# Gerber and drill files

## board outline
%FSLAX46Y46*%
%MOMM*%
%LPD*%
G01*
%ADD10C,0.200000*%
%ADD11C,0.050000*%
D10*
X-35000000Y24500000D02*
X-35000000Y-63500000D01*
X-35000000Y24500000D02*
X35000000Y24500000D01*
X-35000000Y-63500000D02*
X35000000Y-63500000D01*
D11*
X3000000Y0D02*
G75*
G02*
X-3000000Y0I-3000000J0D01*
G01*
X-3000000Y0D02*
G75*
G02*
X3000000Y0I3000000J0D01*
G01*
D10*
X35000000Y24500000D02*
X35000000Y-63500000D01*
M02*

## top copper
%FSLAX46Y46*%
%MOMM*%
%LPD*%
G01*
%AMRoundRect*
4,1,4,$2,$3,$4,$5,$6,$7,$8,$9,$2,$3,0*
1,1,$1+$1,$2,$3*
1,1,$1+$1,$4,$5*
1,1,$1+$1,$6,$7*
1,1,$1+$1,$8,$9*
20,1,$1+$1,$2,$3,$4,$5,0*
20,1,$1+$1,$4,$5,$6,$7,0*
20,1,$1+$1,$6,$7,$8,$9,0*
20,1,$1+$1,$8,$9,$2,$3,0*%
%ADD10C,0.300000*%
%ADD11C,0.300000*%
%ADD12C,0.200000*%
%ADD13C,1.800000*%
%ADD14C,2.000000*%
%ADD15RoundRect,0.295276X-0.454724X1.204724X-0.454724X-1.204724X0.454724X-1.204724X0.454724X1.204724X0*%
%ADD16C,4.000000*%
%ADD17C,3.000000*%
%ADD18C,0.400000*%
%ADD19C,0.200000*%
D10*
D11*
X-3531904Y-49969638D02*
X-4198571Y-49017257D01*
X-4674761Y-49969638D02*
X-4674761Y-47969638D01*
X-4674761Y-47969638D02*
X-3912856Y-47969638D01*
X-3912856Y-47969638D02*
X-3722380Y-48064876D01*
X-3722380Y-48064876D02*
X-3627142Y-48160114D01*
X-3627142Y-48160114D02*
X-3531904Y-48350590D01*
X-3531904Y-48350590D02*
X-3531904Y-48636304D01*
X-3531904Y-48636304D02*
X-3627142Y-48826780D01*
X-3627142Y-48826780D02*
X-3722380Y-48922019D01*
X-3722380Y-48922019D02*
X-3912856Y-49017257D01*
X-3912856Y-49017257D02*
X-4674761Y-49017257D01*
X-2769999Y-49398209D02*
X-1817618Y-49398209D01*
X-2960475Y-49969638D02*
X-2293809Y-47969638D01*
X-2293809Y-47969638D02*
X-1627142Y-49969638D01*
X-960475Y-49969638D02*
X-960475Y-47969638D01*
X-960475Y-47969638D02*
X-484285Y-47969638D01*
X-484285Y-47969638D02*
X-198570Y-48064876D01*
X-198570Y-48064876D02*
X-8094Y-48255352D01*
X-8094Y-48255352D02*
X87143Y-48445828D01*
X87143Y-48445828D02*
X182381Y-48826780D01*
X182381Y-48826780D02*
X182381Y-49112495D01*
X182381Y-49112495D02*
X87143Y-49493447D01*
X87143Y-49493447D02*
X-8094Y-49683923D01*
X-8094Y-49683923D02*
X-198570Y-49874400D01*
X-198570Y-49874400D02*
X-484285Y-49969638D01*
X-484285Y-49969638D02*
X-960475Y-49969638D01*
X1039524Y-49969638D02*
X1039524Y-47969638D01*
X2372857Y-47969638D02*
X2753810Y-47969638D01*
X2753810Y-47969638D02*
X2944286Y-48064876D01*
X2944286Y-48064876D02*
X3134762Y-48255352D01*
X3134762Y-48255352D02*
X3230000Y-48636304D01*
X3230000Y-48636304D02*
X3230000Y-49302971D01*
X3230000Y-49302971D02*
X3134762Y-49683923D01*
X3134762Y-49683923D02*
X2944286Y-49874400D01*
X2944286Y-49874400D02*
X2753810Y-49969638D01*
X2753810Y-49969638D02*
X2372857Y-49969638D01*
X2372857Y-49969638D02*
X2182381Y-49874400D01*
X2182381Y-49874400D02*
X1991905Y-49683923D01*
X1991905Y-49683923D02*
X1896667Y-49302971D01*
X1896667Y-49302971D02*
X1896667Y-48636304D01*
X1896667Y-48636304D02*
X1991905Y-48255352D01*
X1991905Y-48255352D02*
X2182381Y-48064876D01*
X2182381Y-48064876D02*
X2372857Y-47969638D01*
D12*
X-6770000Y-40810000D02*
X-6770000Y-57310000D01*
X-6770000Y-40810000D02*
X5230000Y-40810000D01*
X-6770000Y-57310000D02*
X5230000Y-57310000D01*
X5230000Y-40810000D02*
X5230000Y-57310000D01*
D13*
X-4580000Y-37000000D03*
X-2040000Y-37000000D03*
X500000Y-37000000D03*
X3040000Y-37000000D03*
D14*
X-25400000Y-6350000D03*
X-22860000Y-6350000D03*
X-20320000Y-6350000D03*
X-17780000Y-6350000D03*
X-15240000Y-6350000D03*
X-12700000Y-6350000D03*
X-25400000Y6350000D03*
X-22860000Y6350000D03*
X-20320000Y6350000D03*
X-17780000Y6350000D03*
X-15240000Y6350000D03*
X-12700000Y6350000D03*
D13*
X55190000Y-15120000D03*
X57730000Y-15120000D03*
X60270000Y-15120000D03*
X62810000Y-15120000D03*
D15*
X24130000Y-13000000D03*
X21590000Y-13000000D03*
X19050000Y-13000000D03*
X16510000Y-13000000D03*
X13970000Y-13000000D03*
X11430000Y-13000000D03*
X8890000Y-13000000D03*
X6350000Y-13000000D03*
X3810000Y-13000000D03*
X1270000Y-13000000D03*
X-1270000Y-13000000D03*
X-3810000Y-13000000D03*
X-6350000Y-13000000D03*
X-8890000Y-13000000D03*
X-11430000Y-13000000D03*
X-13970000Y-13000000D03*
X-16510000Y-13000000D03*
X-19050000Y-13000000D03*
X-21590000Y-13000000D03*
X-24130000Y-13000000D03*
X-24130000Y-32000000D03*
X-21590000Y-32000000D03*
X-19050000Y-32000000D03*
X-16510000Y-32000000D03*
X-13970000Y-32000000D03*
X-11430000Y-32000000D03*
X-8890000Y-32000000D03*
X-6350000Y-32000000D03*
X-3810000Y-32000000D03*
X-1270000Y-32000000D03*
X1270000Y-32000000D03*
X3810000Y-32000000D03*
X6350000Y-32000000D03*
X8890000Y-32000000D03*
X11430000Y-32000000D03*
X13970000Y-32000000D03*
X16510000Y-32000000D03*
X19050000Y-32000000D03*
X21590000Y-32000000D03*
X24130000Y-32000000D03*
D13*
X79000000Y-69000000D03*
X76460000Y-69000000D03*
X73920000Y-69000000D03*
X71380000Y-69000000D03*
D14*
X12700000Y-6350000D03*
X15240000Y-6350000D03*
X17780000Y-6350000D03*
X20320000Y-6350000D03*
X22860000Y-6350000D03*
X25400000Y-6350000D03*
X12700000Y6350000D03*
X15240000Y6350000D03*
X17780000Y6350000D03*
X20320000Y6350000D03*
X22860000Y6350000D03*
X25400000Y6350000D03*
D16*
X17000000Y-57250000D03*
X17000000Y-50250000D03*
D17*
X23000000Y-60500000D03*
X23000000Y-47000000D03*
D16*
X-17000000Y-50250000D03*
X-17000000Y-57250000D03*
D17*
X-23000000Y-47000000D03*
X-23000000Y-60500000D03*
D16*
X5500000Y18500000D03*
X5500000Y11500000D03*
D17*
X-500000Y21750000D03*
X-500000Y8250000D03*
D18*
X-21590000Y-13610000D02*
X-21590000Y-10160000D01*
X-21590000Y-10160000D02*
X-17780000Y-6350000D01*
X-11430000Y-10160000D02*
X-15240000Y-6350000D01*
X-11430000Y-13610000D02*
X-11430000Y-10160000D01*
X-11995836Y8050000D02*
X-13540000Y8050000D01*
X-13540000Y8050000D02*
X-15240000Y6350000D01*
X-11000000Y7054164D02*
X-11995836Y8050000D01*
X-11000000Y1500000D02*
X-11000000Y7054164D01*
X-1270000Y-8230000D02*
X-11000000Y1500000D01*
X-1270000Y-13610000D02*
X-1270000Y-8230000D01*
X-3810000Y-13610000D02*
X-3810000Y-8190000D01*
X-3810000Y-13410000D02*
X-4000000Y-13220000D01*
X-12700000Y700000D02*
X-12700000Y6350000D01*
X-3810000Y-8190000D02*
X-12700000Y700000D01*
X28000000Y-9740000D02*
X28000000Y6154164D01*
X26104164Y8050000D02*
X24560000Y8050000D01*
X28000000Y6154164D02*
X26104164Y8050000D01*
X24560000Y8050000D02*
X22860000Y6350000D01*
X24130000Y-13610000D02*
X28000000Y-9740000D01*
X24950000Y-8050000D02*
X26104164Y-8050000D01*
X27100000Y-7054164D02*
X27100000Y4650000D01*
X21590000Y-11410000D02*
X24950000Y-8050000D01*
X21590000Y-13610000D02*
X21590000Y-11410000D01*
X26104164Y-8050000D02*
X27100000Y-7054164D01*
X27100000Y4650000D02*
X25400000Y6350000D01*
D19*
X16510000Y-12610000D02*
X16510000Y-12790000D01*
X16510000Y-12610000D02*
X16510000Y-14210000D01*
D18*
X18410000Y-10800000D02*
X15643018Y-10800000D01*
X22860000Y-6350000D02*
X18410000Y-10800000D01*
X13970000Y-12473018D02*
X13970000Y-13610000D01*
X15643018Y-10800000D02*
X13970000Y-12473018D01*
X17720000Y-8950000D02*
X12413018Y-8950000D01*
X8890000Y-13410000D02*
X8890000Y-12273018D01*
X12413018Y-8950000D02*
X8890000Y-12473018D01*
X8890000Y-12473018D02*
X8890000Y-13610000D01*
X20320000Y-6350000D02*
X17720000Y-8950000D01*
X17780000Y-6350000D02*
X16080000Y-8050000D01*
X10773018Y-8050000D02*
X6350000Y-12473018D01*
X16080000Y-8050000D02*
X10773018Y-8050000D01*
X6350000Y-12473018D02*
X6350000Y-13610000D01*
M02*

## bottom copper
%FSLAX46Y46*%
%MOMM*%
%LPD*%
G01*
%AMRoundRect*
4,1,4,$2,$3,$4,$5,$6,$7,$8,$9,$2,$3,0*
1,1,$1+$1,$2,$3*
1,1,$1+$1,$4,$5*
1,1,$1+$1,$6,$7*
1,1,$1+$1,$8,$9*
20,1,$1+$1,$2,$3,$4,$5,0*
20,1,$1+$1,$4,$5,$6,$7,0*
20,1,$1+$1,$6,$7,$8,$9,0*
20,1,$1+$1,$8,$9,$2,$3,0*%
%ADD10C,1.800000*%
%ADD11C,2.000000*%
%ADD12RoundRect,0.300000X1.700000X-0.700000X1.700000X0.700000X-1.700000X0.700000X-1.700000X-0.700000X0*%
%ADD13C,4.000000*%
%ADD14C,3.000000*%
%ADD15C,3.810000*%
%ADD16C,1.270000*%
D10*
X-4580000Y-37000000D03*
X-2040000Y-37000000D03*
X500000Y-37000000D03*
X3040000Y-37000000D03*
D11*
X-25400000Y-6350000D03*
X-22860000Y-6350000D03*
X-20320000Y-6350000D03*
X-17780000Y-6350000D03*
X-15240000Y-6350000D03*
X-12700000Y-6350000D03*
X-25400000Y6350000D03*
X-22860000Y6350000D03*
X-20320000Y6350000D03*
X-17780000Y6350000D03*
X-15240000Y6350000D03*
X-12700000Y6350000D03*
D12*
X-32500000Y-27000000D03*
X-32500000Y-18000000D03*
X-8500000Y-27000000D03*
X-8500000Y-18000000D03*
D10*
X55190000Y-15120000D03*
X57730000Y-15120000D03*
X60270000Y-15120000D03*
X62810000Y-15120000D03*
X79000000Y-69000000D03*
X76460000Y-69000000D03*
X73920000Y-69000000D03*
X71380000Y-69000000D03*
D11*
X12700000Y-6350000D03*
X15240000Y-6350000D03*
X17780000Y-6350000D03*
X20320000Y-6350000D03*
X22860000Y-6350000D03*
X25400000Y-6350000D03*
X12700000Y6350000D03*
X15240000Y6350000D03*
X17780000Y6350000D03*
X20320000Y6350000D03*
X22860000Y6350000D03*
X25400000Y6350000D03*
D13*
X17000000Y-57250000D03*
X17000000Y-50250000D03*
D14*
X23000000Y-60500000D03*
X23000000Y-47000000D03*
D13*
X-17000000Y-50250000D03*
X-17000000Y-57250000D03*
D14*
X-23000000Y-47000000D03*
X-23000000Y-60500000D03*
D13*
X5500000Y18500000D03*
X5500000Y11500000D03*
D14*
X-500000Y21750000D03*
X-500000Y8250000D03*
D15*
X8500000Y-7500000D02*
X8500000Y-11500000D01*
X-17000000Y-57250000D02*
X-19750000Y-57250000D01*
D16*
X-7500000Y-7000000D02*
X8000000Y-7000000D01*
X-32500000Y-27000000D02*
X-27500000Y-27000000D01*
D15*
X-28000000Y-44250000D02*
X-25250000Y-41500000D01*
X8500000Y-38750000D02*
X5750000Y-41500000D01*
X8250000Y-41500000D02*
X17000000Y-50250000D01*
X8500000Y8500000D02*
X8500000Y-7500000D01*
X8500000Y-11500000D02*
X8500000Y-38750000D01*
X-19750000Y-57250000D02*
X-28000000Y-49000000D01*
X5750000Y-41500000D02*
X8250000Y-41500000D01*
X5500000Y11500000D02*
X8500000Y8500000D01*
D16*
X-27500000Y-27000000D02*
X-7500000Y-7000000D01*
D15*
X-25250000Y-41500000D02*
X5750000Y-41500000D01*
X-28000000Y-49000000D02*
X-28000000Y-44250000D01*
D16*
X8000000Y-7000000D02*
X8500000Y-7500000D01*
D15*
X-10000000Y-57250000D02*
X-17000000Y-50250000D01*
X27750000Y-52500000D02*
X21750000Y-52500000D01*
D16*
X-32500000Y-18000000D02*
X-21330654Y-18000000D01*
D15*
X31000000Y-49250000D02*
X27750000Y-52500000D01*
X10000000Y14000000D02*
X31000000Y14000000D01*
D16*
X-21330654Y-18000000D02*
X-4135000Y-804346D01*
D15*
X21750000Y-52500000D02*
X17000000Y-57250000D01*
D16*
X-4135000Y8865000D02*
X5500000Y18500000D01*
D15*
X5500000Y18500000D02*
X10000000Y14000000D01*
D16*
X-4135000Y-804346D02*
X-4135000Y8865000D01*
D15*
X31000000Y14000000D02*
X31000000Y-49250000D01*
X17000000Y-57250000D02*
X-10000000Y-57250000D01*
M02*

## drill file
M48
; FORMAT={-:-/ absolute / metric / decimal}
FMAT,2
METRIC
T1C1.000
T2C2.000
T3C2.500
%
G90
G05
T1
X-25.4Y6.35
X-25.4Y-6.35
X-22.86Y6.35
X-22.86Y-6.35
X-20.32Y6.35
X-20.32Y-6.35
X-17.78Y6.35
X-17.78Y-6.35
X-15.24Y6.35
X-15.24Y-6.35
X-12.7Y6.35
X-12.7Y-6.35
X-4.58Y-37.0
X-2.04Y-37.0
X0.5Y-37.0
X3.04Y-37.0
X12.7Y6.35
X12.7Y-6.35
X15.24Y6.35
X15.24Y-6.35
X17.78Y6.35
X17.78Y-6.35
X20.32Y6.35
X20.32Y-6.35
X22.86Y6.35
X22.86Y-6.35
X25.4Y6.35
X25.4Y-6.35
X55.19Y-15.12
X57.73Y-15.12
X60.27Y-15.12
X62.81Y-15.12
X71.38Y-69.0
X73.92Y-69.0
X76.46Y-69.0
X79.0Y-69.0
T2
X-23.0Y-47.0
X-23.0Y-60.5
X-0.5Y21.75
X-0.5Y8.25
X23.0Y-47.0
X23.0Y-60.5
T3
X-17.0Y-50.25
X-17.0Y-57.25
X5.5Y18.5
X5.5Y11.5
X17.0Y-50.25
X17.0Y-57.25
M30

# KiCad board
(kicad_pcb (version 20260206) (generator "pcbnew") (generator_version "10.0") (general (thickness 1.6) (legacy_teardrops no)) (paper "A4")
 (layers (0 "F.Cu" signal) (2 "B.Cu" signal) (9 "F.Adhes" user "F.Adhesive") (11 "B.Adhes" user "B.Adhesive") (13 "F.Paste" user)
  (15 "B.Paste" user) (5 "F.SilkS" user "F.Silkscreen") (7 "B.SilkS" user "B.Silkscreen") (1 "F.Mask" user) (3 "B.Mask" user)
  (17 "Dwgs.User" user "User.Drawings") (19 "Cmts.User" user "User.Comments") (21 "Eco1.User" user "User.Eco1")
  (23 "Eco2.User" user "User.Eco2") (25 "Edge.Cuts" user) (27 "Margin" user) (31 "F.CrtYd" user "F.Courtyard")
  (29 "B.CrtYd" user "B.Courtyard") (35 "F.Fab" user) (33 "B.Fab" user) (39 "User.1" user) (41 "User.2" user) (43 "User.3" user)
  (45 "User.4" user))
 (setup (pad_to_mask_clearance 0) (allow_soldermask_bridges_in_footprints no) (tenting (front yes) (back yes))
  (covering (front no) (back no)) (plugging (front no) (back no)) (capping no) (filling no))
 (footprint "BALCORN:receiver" (layer "F.Cu") (at -0.77 49.06)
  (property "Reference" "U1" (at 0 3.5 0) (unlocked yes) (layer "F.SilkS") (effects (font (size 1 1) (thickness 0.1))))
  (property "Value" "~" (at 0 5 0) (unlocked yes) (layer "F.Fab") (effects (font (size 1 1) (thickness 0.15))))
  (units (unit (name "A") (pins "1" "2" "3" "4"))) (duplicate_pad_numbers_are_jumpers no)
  (fp_line (start -6 -8.25) (end -6 8.25) (stroke (width 0.2) (type default)) (layer "F.Cu"))
  (fp_line (start -6 -8.25) (end 6 -8.25) (stroke (width 0.2) (type default)) (layer "F.Cu"))
  (fp_line (start -6 8.25) (end 6 8.25) (stroke (width 0.2) (type default)) (layer "F.Cu"))
  (fp_line (start 6 -8.25) (end 6 8.25) (stroke (width 0.2) (type default)) (layer "F.Cu"))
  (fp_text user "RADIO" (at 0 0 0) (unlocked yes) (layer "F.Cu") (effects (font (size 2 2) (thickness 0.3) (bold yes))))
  (pad "1" thru_hole circle (at -3.81 -12.06) (size 1.8 1.8) (drill 1) (layers "*.Cu" "*.Mask") (remove_unused_layers no)
   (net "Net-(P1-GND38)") (thermal_bridge_angle 90))
  (pad "2" thru_hole circle (at -1.27 -12.06) (size 1.8 1.8) (drill 1) (layers "*.Cu" "*.Mask") (remove_unused_layers no)
   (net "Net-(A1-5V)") (thermal_bridge_angle 90))
  (pad "3" thru_hole circle (at 1.27 -12.06) (size 1.8 1.8) (drill 1) (layers "*.Cu" "*.Mask") (remove_unused_layers no)
   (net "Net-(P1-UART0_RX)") (thermal_bridge_angle 90))
  (pad "4" thru_hole circle (at 3.81 -12.06) (size 1.8 1.8) (drill 1) (layers "*.Cu" "*.Mask") (remove_unused_layers no)
   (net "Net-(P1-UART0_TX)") (thermal_bridge_angle 90)))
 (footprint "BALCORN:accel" (layer "F.Cu") (at -19.05 0 90)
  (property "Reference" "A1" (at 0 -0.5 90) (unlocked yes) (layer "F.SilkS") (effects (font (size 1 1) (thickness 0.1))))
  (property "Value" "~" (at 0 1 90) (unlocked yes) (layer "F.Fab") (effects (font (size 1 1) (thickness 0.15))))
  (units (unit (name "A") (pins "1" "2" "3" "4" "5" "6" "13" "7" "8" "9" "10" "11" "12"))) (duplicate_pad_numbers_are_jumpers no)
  (pad "1" thru_hole circle (at -6.35 -6.35 90) (size 2 2) (drill 1) (layers "*.Cu" "*.Mask") (remove_unused_layers no) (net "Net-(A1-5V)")
   (thermal_bridge_angle 90))
  (pad "2" thru_hole circle (at -6.35 -3.81 90) (size 2 2) (drill 1) (layers "*.Cu" "*.Mask") (remove_unused_layers no)
   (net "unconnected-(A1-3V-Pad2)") (thermal_bridge_angle 90))
  (pad "3" thru_hole circle (at -6.35 -1.27 90) (size 2 2) (drill 1) (layers "*.Cu" "*.Mask") (remove_unused_layers no)
   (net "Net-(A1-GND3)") (thermal_bridge_angle 90))
  (pad "4" thru_hole circle (at -6.35 1.27 90) (size 2 2) (drill 1) (layers "*.Cu" "*.Mask") (remove_unused_layers no) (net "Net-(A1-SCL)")
   (thermal_bridge_angle 90))
  (pad "5" thru_hole circle (at -6.35 3.81 90) (size 2 2) (drill 1) (layers "*.Cu" "*.Mask") (remove_unused_layers no) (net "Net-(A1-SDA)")
   (thermal_bridge_angle 90))
  (pad "6" thru_hole circle (at -6.35 6.35 90) (size 2 2) (drill 1) (layers "*.Cu" "*.Mask") (remove_unused_layers no)
   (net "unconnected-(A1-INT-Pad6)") (thermal_bridge_angle 90))
  (pad "7" thru_hole circle (at 6.35 -6.35 90) (size 2 2) (drill 1) (layers "*.Cu" "*.Mask") (remove_unused_layers no)
   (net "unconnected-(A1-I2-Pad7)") (thermal_bridge_angle 90))
  (pad "8" thru_hole circle (at 6.35 -3.81 90) (size 2 2) (drill 1) (layers "*.Cu" "*.Mask") (remove_unused_layers no)
   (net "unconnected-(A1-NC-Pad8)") (thermal_bridge_angle 90))
  (pad "9" thru_hole circle (at 6.35 -1.27 90) (size 2 2) (drill 1) (layers "*.Cu" "*.Mask") (remove_unused_layers no)
   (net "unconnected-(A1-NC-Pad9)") (thermal_bridge_angle 90))
  (pad "10" thru_hole circle (at 6.35 1.27 90) (size 2 2) (drill 1) (layers "*.Cu" "*.Mask") (remove_unused_layers no)
   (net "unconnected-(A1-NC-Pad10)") (thermal_bridge_angle 90))
  (pad "11" thru_hole circle (at 6.35 3.81 90) (size 2 2) (drill 1) (layers "*.Cu" "*.Mask") (remove_unused_layers no) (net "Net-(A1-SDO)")
   (thermal_bridge_angle 90))
  (pad "12" thru_hole circle (at 6.35 6.35 90) (size 2 2) (drill 1) (layers "*.Cu" "*.Mask") (remove_unused_layers no) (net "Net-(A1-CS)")
   (thermal_bridge_angle 90)))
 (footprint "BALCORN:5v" (layer "F.Cu") (at -20.5 22.5 90)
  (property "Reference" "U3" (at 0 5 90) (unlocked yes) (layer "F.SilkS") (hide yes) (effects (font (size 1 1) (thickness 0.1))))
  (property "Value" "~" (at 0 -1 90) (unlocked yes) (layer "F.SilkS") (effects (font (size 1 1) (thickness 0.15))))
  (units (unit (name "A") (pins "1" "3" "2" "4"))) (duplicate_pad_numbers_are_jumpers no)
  (pad "1" smd roundrect (at -4.5 -12 90) (size 2 4) (layers "B.Cu" "B.Mask") (roundrect_rratio 0.15) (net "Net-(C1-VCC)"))
  (pad "2" smd roundrect (at 4.5 -12 90) (size 2 4) (layers "B.Cu" "B.Mask") (roundrect_rratio 0.15) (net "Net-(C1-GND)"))
  (pad "3" smd roundrect (at -4.5 12 90) (size 2 4) (layers "B.Cu" "B.Mask") (roundrect_rratio 0.15) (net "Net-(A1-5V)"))
  (pad "4" smd roundrect (at 4.5 12 90) (size 2 4) (layers "B.Cu" "B.Mask") (roundrect_rratio 0.15) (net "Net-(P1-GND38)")))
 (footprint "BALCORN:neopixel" (layer "F.Cu") (at 59 15.12)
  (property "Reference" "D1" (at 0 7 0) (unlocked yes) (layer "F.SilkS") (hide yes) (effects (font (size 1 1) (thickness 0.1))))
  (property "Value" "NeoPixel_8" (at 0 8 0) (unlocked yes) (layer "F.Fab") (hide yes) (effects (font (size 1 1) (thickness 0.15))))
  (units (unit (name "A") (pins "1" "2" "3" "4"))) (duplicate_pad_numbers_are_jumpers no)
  (pad "1" thru_hole circle (at -3.81 0) (size 1.8 1.8) (drill 1) (layers "*.Cu" "*.Mask") (remove_unused_layers no)
   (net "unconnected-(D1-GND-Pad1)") (thermal_bridge_angle 90))
  (pad "2" thru_hole circle (at -1.27 0) (size 1.8 1.8) (drill 1) (layers "*.Cu" "*.Mask") (remove_unused_layers no)
   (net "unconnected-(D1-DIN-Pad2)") (thermal_bridge_angle 90))
  (pad "3" thru_hole circle (at 1.27 0) (size 1.8 1.8) (drill 1) (layers "*.Cu" "*.Mask") (remove_unused_layers no) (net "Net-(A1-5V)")
   (thermal_bridge_angle 90))
  (pad "4" thru_hole circle (at 3.81 0) (size 1.8 1.8) (drill 1) (layers "*.Cu" "*.Mask") (remove_unused_layers no) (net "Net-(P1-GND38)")
   (thermal_bridge_angle 90)))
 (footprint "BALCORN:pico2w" (layer "F.Cu") (at 0 22.5 -90)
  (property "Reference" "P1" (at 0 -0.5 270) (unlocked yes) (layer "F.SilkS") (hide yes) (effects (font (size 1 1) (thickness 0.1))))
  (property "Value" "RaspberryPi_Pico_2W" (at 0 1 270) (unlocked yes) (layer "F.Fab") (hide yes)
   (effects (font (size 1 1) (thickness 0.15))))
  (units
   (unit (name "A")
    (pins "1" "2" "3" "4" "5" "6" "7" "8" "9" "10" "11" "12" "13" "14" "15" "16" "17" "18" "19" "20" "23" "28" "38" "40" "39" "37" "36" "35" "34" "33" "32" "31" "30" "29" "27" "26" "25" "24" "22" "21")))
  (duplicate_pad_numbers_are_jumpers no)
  (pad "1" smd roundrect (at -8.89 -24.13 270) (size 3 1.5) (drill (offset -0.61 0)) (layers "F.Cu" "F.Mask")
   (roundrect_rratio 0.1968503937) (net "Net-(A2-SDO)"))
  (pad "2" smd roundrect (at -8.89 -21.59 270) (size 3 1.5) (drill (offset -0.61 0)) (layers "F.Cu" "F.Mask")
   (roundrect_rratio 0.1968503937) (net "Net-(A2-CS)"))
  (pad "3" smd roundrect (at -8.89 -19.05 270) (size 3 1.5) (drill (offset -0.61 0)) (layers "F.Cu" "F.Mask")
   (roundrect_rratio 0.1968503937) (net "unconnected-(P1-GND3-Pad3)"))
  (pad "4" smd roundrect (at -8.89 -16.51 270) (size 3 1.5) (drill (offset -0.61 0)) (layers "F.Cu" "F.Mask")
   (roundrect_rratio 0.1968503937) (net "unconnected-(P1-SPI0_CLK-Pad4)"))
  (pad "5" smd roundrect (at -8.89 -13.97 270) (size 3 1.5) (drill (offset -0.61 0)) (layers "F.Cu" "F.Mask")
   (roundrect_rratio 0.1968503937) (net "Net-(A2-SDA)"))
  (pad "6" smd roundrect (at -8.89 -11.43 270) (size 3 1.5) (drill (offset -0.61 0)) (layers "F.Cu" "F.Mask")
   (roundrect_rratio 0.1968503937) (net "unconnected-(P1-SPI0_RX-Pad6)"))
  (pad "7" smd roundrect (at -8.89 -8.89 270) (size 3 1.5) (drill (offset -0.61 0)) (layers "F.Cu" "F.Mask") (roundrect_rratio 0.1968503937)
   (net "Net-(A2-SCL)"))
  (pad "8" smd roundrect (at -8.89 -6.35 270) (size 3 1.5) (drill (offset -0.61 0)) (layers "F.Cu" "F.Mask") (roundrect_rratio 0.1968503937)
   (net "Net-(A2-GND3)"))
  (pad "9" smd roundrect (at -8.89 -3.81 270) (size 3 1.5) (drill (offset -0.61 0)) (layers "F.Cu" "F.Mask") (roundrect_rratio 0.1968503937)
   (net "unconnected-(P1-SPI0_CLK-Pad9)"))
  (pad "10" smd roundrect (at -8.89 -1.27 270) (size 3 1.5) (drill (offset -0.61 0)) (layers "F.Cu" "F.Mask")
   (roundrect_rratio 0.1968503937) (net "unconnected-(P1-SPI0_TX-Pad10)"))
  (pad "11" smd roundrect (at -8.89 1.27 270) (size 3 1.5) (drill (offset -0.61 0)) (layers "F.Cu" "F.Mask") (roundrect_rratio 0.1968503937)
   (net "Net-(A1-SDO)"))
  (pad "12" smd roundrect (at -8.89 3.81 270) (size 3 1.5) (drill (offset -0.61 0)) (layers "F.Cu" "F.Mask") (roundrect_rratio 0.1968503937)
   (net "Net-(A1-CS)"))
  (pad "13" smd roundrect (at -8.89 6.35 270) (size 3 1.5) (drill (offset -0.61 0)) (layers "F.Cu" "F.Mask") (roundrect_rratio 0.1968503937)
   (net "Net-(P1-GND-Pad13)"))
  (pad "14" smd roundrect (at -8.89 8.89 270) (size 3 1.5) (drill (offset -0.61 0)) (layers "F.Cu" "F.Mask") (roundrect_rratio 0.1968503937)
   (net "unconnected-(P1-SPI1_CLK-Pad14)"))
  (pad "15" smd roundrect (at -8.89 11.43 270) (size 3 1.5) (drill (offset -0.61 0)) (layers "F.Cu" "F.Mask")
   (roundrect_rratio 0.1968503937) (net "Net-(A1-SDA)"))
  (pad "16" smd roundrect (at -8.89 13.97 270) (size 3 1.5) (drill (offset -0.61 0)) (layers "F.Cu" "F.Mask")
   (roundrect_rratio 0.1968503937) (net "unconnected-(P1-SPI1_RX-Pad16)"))
  (pad "17" smd roundrect (at -8.89 16.51 270) (size 3 1.5) (drill (offset -0.61 0)) (layers "F.Cu" "F.Mask")
   (roundrect_rratio 0.1968503937) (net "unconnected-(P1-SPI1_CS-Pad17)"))
  (pad "18" smd roundrect (at -8.89 19.05 270) (size 3 1.5) (drill (offset -0.61 0)) (layers "F.Cu" "F.Mask")
   (roundrect_rratio 0.1968503937) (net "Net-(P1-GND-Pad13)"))
  (pad "19" smd roundrect (at -8.89 21.59 270) (size 3 1.5) (drill (offset -0.61 0)) (layers "F.Cu" "F.Mask")
   (roundrect_rratio 0.1968503937) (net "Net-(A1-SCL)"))
  (pad "20" smd roundrect (at -8.89 24.13 270) (size 3 1.5) (drill (offset -0.61 0)) (layers "F.Cu" "F.Mask")
   (roundrect_rratio 0.1968503937) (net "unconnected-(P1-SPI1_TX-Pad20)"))
  (pad "21" smd roundrect (at 8.89 24.13 270) (size 3 1.5) (drill (offset 0.61 0)) (layers "F.Cu" "F.Mask") (roundrect_rratio 0.1968503937)
   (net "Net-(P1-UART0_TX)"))
  (pad "22" smd roundrect (at 8.89 21.59 270) (size 3 1.5) (drill (offset 0.61 0)) (layers "F.Cu" "F.Mask") (roundrect_rratio 0.1968503937)
   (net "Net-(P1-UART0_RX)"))
  (pad "23" smd roundrect (at 8.89 19.05 270) (size 3 1.5) (drill (offset 0.61 0)) (layers "F.Cu" "F.Mask") (roundrect_rratio 0.1968503937)
   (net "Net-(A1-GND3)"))
  (pad "24" smd roundrect (at 8.89 16.51 270) (size 3 1.5) (drill (offset 0.61 0)) (layers "F.Cu" "F.Mask") (roundrect_rratio 0.1968503937)
   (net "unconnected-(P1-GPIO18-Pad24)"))
  (pad "25" smd roundrect (at 8.89 13.97 270) (size 3 1.5) (drill (offset 0.61 0)) (layers "F.Cu" "F.Mask") (roundrect_rratio 0.1968503937)
   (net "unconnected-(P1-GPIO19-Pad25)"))
  (pad "26" smd roundrect (at 8.89 11.43 270) (size 3 1.5) (drill (offset 0.61 0)) (layers "F.Cu" "F.Mask") (roundrect_rratio 0.1968503937)
   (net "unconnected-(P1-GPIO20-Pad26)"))
  (pad "27" smd roundrect (at 8.89 8.89 270) (size 3 1.5) (drill (offset 0.61 0)) (layers "F.Cu" "F.Mask") (roundrect_rratio 0.1968503937)
   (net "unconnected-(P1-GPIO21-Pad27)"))
  (pad "28" smd roundrect (at 8.89 6.35 270) (size 3 1.5) (drill (offset 0.61 0)) (layers "F.Cu" "F.Mask") (roundrect_rratio 0.1968503937)
   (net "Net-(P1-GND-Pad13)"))
  (pad "29" smd roundrect (at 8.89 3.81 270) (size 3 1.5) (drill (offset 0.61 0)) (layers "F.Cu" "F.Mask") (roundrect_rratio 0.1968503937)
   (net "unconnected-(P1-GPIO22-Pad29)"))
  (pad "30" smd roundrect (at 8.89 1.27 270) (size 3 1.5) (drill (offset 0.61 0)) (layers "F.Cu" "F.Mask") (roundrect_rratio 0.1968503937)
   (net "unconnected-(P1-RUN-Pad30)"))
  (pad "31" smd roundrect (at 8.89 -1.27 270) (size 3 1.5) (drill (offset 0.61 0)) (layers "F.Cu" "F.Mask") (roundrect_rratio 0.1968503937)
   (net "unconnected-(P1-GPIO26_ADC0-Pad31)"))
  (pad "32" smd roundrect (at 8.89 -3.81 270) (size 3 1.5) (drill (offset 0.61 0)) (layers "F.Cu" "F.Mask") (roundrect_rratio 0.1968503937)
   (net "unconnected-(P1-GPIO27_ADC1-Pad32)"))
  (pad "33" smd roundrect (at 8.89 -6.35 270) (size 3 1.5) (drill (offset 0.61 0)) (layers "F.Cu" "F.Mask") (roundrect_rratio 0.1968503937)
   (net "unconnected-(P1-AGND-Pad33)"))
  (pad "34" smd roundrect (at 8.89 -8.89 270) (size 3 1.5) (drill (offset 0.61 0)) (layers "F.Cu" "F.Mask") (roundrect_rratio 0.1968503937)
   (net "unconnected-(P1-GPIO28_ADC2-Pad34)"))
  (pad "35" smd roundrect (at 8.89 -11.43 270) (size 3 1.5) (drill (offset 0.61 0)) (layers "F.Cu" "F.Mask") (roundrect_rratio 0.1968503937)
   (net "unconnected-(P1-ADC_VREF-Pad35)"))
  (pad "36" smd roundrect (at 8.89 -13.97 270) (size 3 1.5) (drill (offset 0.61 0)) (layers "F.Cu" "F.Mask") (roundrect_rratio 0.1968503937)
   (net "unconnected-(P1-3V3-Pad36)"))
  (pad "37" smd roundrect (at 8.89 -16.51 270) (size 3 1.5) (drill (offset 0.61 0)) (layers "F.Cu" "F.Mask") (roundrect_rratio 0.1968503937)
   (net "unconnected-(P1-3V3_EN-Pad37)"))
  (pad "38" smd roundrect (at 8.89 -19.05 270) (size 3 1.5) (drill (offset 0.61 0)) (layers "F.Cu" "F.Mask") (roundrect_rratio 0.1968503937)
   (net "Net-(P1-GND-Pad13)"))
  (pad "39" smd roundrect (at 8.89 -21.59 270) (size 3 1.5) (drill (offset 0.61 0)) (layers "F.Cu" "F.Mask") (roundrect_rratio 0.1968503937)
   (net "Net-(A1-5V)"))
  (pad "40" smd roundrect (at 8.89 -24.13 270) (size 3 1.5) (drill (offset 0.61 0)) (layers "F.Cu" "F.Mask") (roundrect_rratio 0.1968503937)
   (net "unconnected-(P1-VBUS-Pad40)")))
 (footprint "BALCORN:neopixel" (layer "F.Cu") (at 75.19 69 180)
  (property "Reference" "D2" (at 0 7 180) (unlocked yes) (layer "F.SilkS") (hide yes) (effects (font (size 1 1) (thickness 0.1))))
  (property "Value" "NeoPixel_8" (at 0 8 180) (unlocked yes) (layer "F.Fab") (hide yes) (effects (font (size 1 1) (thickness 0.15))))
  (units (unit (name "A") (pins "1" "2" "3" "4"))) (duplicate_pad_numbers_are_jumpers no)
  (pad "1" thru_hole circle (at -3.81 0 180) (size 1.8 1.8) (drill 1) (layers "*.Cu" "*.Mask") (remove_unused_layers no)
   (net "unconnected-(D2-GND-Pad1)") (thermal_bridge_angle 90))
  (pad "2" thru_hole circle (at -1.27 0 180) (size 1.8 1.8) (drill 1) (layers "*.Cu" "*.Mask") (remove_unused_layers no)
   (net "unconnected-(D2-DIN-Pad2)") (thermal_bridge_angle 90))
  (pad "3" thru_hole circle (at 1.27 0 180) (size 1.8 1.8) (drill 1) (layers "*.Cu" "*.Mask") (remove_unused_layers no) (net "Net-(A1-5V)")
   (thermal_bridge_angle 90))
  (pad "4" thru_hole circle (at 3.81 0 180) (size 1.8 1.8) (drill 1) (layers "*.Cu" "*.Mask") (remove_unused_layers no)
   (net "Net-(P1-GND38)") (thermal_bridge_angle 90)))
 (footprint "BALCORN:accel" (layer "F.Cu") (at 19.05 0 90)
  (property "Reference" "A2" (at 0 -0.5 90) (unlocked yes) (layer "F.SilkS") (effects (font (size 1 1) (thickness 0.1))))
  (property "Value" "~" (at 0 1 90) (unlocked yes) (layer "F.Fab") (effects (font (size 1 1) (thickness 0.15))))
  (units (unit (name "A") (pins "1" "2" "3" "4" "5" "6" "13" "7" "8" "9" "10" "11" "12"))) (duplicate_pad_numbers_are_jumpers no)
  (pad "1" thru_hole circle (at -6.35 -6.35 90) (size 2 2) (drill 1) (layers "*.Cu" "*.Mask") (remove_unused_layers no) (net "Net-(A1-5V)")
   (thermal_bridge_angle 90))
  (pad "2" thru_hole circle (at -6.35 -3.81 90) (size 2 2) (drill 1) (layers "*.Cu" "*.Mask") (remove_unused_layers no)
   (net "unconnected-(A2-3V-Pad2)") (thermal_bridge_angle 90))
  (pad "3" thru_hole circle (at -6.35 -1.27 90) (size 2 2) (drill 1) (layers "*.Cu" "*.Mask") (remove_unused_layers no)
   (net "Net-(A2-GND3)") (thermal_bridge_angle 90))
  (pad "4" thru_hole circle (at -6.35 1.27 90) (size 2 2) (drill 1) (layers "*.Cu" "*.Mask") (remove_unused_layers no) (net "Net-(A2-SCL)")
   (thermal_bridge_angle 90))
  (pad "5" thru_hole circle (at -6.35 3.81 90) (size 2 2) (drill 1) (layers "*.Cu" "*.Mask") (remove_unused_layers no) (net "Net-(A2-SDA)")
   (thermal_bridge_angle 90))
  (pad "6" thru_hole circle (at -6.35 6.35 90) (size 2 2) (drill 1) (layers "*.Cu" "*.Mask") (remove_unused_layers no)
   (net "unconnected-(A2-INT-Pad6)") (thermal_bridge_angle 90))
  (pad "7" thru_hole circle (at 6.35 -6.35 90) (size 2 2) (drill 1) (layers "*.Cu" "*.Mask") (remove_unused_layers no)
   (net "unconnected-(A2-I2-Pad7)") (thermal_bridge_angle 90))
  (pad "8" thru_hole circle (at 6.35 -3.81 90) (size 2 2) (drill 1) (layers "*.Cu" "*.Mask") (remove_unused_layers no)
   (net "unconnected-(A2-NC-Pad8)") (thermal_bridge_angle 90))
  (pad "9" thru_hole circle (at 6.35 -1.27 90) (size 2 2) (drill 1) (layers "*.Cu" "*.Mask") (remove_unused_layers no)
   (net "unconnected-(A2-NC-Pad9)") (thermal_bridge_angle 90))
  (pad "10" thru_hole circle (at 6.35 1.27 90) (size 2 2) (drill 1) (layers "*.Cu" "*.Mask") (remove_unused_layers no)
   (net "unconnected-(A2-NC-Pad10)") (thermal_bridge_angle 90))
  (pad "11" thru_hole circle (at 6.35 3.81 90) (size 2 2) (drill 1) (layers "*.Cu" "*.Mask") (remove_unused_layers no) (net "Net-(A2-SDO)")
   (thermal_bridge_angle 90))
  (pad "12" thru_hole circle (at 6.35 6.35 90) (size 2 2) (drill 1) (layers "*.Cu" "*.Mask") (remove_unused_layers no) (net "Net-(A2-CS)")
   (thermal_bridge_angle 90)))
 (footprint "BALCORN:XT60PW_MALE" (layer "B.Cu") (at 24.175 53.75 90)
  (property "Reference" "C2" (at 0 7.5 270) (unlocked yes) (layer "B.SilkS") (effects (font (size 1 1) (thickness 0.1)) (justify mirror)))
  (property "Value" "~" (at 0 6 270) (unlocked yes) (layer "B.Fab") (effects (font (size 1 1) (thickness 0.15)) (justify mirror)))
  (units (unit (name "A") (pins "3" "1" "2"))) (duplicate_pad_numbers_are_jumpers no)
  (pad "1" thru_hole circle (at -3.5 -7.175 90) (size 4 4) (drill 2.5) (layers "*.Cu" "*.Mask") (remove_unused_layers no)
   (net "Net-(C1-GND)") (thermal_bridge_angle 90))
  (pad "2" thru_hole circle (at 3.5 -7.175 90) (size 4 4) (drill 2.5) (layers "*.Cu" "*.Mask") (remove_unused_layers no)
   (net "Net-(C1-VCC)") (thermal_bridge_angle 90))
  (pad "3" thru_hole circle (at -6.75 -1.175 90) (size 3 3) (drill 2) (layers "*.Cu" "*.Mask") (remove_unused_layers no)
   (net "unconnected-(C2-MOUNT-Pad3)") (thermal_bridge_angle 90))
  (pad "4" thru_hole circle (at 6.75 -1.175 90) (size 3 3) (drill 2) (layers "*.Cu" "*.Mask") (remove_unused_layers no)
   (thermal_bridge_angle 90)))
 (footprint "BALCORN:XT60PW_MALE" (layer "B.Cu") (at -24.175 53.75 -90)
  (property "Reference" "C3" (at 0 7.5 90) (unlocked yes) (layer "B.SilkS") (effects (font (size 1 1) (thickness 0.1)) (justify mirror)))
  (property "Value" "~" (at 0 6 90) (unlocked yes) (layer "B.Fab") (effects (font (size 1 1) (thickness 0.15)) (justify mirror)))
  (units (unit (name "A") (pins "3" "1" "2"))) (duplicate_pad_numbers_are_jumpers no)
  (pad "1" thru_hole circle (at -3.5 -7.175 270) (size 4 4) (drill 2.5) (layers "*.Cu" "*.Mask") (remove_unused_layers no)
   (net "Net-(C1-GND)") (thermal_bridge_angle 90))
  (pad "2" thru_hole circle (at 3.5 -7.175 270) (size 4 4) (drill 2.5) (layers "*.Cu" "*.Mask") (remove_unused_layers no)
   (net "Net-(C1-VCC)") (thermal_bridge_angle 90))
  (pad "3" thru_hole circle (at -6.75 -1.175 270) (size 3 3) (drill 2) (layers "*.Cu" "*.Mask") (remove_unused_layers no)
   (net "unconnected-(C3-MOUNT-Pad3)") (thermal_bridge_angle 90))
  (pad "4" thru_hole circle (at 6.75 -1.175 270) (size 3 3) (drill 2) (layers "*.Cu" "*.Mask") (remove_unused_layers no)
   (thermal_bridge_angle 90)))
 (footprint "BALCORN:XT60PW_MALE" (layer "B.Cu") (at -1.675 -15 -90)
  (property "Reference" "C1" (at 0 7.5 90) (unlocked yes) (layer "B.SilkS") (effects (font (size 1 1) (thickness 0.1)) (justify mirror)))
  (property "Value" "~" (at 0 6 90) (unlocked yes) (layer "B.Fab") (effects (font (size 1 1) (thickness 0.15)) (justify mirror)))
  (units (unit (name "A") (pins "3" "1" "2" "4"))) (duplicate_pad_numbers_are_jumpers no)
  (pad "1" thru_hole circle (at -3.5 -7.175 270) (size 4 4) (drill 2.5) (layers "*.Cu" "*.Mask") (remove_unused_layers no)
   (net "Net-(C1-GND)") (thermal_bridge_angle 90))
  (pad "2" thru_hole circle (at 3.5 -7.175 270) (size 4 4) (drill 2.5) (layers "*.Cu" "*.Mask") (remove_unused_layers no)
   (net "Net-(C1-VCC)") (thermal_bridge_angle 90))
  (pad "3" thru_hole circle (at -6.75 -1.175 270) (size 3 3) (drill 2) (layers "*.Cu" "*.Mask") (remove_unused_layers no)
   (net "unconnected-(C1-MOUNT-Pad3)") (thermal_bridge_angle 90))
  (pad "4" thru_hole circle (at 6.75 -1.175 270) (size 3 3) (drill 2) (layers "*.Cu" "*.Mask") (remove_unused_layers no)
   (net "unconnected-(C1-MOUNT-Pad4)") (thermal_bridge_angle 90)))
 (gr_line (start -35 -24.5) (end -35 63.5) (stroke (width 0.2) (type default)) (layer "Edge.Cuts"))
 (gr_line (start -35 -24.5) (end 35 -24.5) (stroke (width 0.2) (type default)) (layer "Edge.Cuts"))
 (gr_line (start -35 63.5) (end 35 63.5) (stroke (width 0.2) (type default)) (layer "Edge.Cuts"))
 (gr_circle (center 0 0) (end 3 0) (stroke (width 0.05) (type default)) (fill no) (layer "Edge.Cuts"))
 (gr_line (start 35 -24.5) (end 35 63.5) (stroke (width 0.2) (type default)) (layer "Edge.Cuts"))
 (segment (start -21.59 13.61) (end -21.59 10.16) (width 0.4) (layer "F.Cu") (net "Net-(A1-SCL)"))
 (segment (start -21.59 10.16) (end -17.78 6.35) (width 0.4) (layer "F.Cu") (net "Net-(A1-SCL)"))
 (segment (start -11.43 10.16) (end -15.24 6.35) (width 0.4) (layer "F.Cu") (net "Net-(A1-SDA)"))
 (segment (start -11.43 13.61) (end -11.43 10.16) (width 0.4) (layer "F.Cu") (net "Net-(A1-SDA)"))
 (segment (start -11.995836 -8.05) (end -13.54 -8.05) (width 0.4) (layer "F.Cu") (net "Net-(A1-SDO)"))
 (segment (start -13.54 -8.05) (end -15.24 -6.35) (width 0.4) (layer "F.Cu") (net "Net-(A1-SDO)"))
 (segment (start -11 -7.054164) (end -11.995836 -8.05) (width 0.4) (layer "F.Cu") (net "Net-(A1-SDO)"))
 (segment (start -11 -1.5) (end -11 -7.054164) (width 0.4) (layer "F.Cu") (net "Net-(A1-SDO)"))
 (segment (start -1.27 8.23) (end -11 -1.5) (width 0.4) (layer "F.Cu") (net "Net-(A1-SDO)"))
 (segment (start -1.27 13.61) (end -1.27 8.23) (width 0.4) (layer "F.Cu") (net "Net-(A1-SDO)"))
 (segment (start -3.81 13.61) (end -3.81 8.19) (width 0.4) (layer "F.Cu") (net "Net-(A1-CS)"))
 (segment (start -3.81 13.41) (end -4 13.22) (width 0.4) (layer "F.Cu") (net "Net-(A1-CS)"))
 (segment (start -12.7 -0.7) (end -12.7 -6.35) (width 0.4) (layer "F.Cu") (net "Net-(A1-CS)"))
 (segment (start -3.81 8.19) (end -12.7 -0.7) (width 0.4) (layer "F.Cu") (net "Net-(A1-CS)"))
 (segment (start 8.5 7.5) (end 8.5 11.5) (width 3.81) (layer "B.Cu") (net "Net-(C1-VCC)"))
 (segment (start -17 57.25) (end -19.75 57.25) (width 3.81) (layer "B.Cu") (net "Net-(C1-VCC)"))
 (segment (start -7.5 7) (end 8 7) (width 1.27) (layer "B.Cu") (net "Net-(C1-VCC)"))
 (segment (start -32.5 27) (end -27.5 27) (width 1.27) (layer "B.Cu") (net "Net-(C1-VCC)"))
 (segment (start -28 44.25) (end -25.25 41.5) (width 3.81) (layer "B.Cu") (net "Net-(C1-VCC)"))
 (segment (start 8.5 38.75) (end 5.75 41.5) (width 3.81) (layer "B.Cu") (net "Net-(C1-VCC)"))
 (segment (start 8.25 41.5) (end 17 50.25) (width 3.81) (layer "B.Cu") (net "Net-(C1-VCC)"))
 (segment (start 8.5 -8.5) (end 8.5 7.5) (width 3.81) (layer "B.Cu") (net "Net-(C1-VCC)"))
 (segment (start 8.5 11.5) (end 8.5 38.75) (width 3.81) (layer "B.Cu") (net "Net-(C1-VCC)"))
 (segment (start -19.75 57.25) (end -28 49) (width 3.81) (layer "B.Cu") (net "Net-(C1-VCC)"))
 (segment (start 5.75 41.5) (end 8.25 41.5) (width 3.81) (layer "B.Cu") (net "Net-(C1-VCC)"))
 (segment (start 5.5 -11.5) (end 8.5 -8.5) (width 3.81) (layer "B.Cu") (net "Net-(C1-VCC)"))
 (segment (start -27.5 27) (end -7.5 7) (width 1.27) (layer "B.Cu") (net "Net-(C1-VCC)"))
 (segment (start -25.25 41.5) (end 5.75 41.5) (width 3.81) (layer "B.Cu") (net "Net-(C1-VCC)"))
 (segment (start -28 49) (end -28 44.25) (width 3.81) (layer "B.Cu") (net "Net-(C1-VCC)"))
 (segment (start 8 7) (end 8.5 7.5) (width 1.27) (layer "B.Cu") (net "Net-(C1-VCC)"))
 (segment (start -10 57.25) (end -17 50.25) (width 3.81) (layer "B.Cu") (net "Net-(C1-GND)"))
 (segment (start 27.75 52.5) (end 21.75 52.5) (width 3.81) (layer "B.Cu") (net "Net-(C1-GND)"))
 (segment (start -32.5 18) (end -21.330654 18) (width 1.27) (layer "B.Cu") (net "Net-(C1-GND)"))
 (segment (start 31 49.25) (end 27.75 52.5) (width 3.81) (layer "B.Cu") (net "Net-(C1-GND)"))
 (segment (start 10 -14) (end 31 -14) (width 3.81) (layer "B.Cu") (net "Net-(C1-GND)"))
 (segment (start -21.330654 18) (end -4.135 0.804346) (width 1.27) (layer "B.Cu") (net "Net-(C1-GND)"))
 (segment (start 21.75 52.5) (end 17 57.25) (width 3.81) (layer "B.Cu") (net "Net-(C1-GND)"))
 (segment (start -4.135 -8.865) (end 5.5 -18.5) (width 1.27) (layer "B.Cu") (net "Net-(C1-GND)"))
 (segment (start 5.5 -18.5) (end 10 -14) (width 3.81) (layer "B.Cu") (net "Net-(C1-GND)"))
 (segment (start -4.135 0.804346) (end -4.135 -8.865) (width 1.27) (layer "B.Cu") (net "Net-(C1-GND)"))
 (segment (start 31 -14) (end 31 49.25) (width 3.81) (layer "B.Cu") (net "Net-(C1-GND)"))
 (segment (start 17 57.25) (end -10 57.25) (width 3.81) (layer "B.Cu") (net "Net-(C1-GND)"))
 (segment (start 28 9.74) (end 28 -6.154164) (width 0.4) (layer "F.Cu") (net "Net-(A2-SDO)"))
 (segment (start 26.104164 -8.05) (end 24.56 -8.05) (width 0.4) (layer "F.Cu") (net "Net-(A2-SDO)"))
 (segment (start 28 -6.154164) (end 26.104164 -8.05) (width 0.4) (layer "F.Cu") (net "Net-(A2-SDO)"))
 (segment (start 24.56 -8.05) (end 22.86 -6.35) (width 0.4) (layer "F.Cu") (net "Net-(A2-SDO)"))
 (segment (start 24.13 13.61) (end 28 9.74) (width 0.4) (layer "F.Cu") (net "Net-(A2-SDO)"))
 (segment (start 24.95 8.05) (end 26.104164 8.05) (width 0.4) (layer "F.Cu") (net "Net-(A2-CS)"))
 (segment (start 27.1 7.054164) (end 27.1 -4.65) (width 0.4) (layer "F.Cu") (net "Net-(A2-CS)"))
 (segment (start 21.59 11.41) (end 24.95 8.05) (width 0.4) (layer "F.Cu") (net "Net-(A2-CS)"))
 (segment (start 21.59 13.61) (end 21.59 11.41) (width 0.4) (layer "F.Cu") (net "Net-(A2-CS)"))
 (segment (start 26.104164 8.05) (end 27.1 7.054164) (width 0.4) (layer "F.Cu") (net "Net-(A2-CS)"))
 (segment (start 27.1 -4.65) (end 25.4 -6.35) (width 0.4) (layer "F.Cu") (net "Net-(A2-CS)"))
 (segment (start 16.51 12.61) (end 16.51 12.79) (width 0.2) (layer "F.Cu") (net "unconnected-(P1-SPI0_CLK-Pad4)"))
 (segment (start 16.51 12.61) (end 16.51 14.21) (width 0.2) (layer "F.Cu") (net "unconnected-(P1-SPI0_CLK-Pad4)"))
 (segment (start 18.41 10.8) (end 15.643018 10.8) (width 0.4) (layer "F.Cu") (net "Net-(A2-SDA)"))
 (segment (start 22.86 6.35) (end 18.41 10.8) (width 0.4) (layer "F.Cu") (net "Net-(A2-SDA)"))
 (segment (start 13.97 12.473018) (end 13.97 13.61) (width 0.4) (layer "F.Cu") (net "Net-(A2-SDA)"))
 (segment (start 15.643018 10.8) (end 13.97 12.473018) (width 0.4) (layer "F.Cu") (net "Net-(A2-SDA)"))
 (segment (start 17.72 8.95) (end 12.413018 8.95) (width 0.4) (layer "F.Cu") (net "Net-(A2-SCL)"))
 (segment (start 8.89 13.41) (end 8.89 12.273018) (width 0.4) (layer "F.Cu") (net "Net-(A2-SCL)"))
 (segment (start 12.413018 8.95) (end 8.89 12.473018) (width 0.4) (layer "F.Cu") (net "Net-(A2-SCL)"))
 (segment (start 8.89 12.473018) (end 8.89 13.61) (width 0.4) (layer "F.Cu") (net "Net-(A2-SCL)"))
 (segment (start 20.32 6.35) (end 17.72 8.95) (width 0.4) (layer "F.Cu") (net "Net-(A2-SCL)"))
 (segment (start 17.78 6.35) (end 16.08 8.05) (width 0.4) (layer "F.Cu") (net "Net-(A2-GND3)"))
 (segment (start 10.773018 8.05) (end 6.35 12.473018) (width 0.4) (layer "F.Cu") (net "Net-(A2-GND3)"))
 (segment (start 16.08 8.05) (end 10.773018 8.05) (width 0.4) (layer "F.Cu") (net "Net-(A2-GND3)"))
 (segment (start 6.35 12.473018) (end 6.35 13.61) (width 0.4) (layer "F.Cu") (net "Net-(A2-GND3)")))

